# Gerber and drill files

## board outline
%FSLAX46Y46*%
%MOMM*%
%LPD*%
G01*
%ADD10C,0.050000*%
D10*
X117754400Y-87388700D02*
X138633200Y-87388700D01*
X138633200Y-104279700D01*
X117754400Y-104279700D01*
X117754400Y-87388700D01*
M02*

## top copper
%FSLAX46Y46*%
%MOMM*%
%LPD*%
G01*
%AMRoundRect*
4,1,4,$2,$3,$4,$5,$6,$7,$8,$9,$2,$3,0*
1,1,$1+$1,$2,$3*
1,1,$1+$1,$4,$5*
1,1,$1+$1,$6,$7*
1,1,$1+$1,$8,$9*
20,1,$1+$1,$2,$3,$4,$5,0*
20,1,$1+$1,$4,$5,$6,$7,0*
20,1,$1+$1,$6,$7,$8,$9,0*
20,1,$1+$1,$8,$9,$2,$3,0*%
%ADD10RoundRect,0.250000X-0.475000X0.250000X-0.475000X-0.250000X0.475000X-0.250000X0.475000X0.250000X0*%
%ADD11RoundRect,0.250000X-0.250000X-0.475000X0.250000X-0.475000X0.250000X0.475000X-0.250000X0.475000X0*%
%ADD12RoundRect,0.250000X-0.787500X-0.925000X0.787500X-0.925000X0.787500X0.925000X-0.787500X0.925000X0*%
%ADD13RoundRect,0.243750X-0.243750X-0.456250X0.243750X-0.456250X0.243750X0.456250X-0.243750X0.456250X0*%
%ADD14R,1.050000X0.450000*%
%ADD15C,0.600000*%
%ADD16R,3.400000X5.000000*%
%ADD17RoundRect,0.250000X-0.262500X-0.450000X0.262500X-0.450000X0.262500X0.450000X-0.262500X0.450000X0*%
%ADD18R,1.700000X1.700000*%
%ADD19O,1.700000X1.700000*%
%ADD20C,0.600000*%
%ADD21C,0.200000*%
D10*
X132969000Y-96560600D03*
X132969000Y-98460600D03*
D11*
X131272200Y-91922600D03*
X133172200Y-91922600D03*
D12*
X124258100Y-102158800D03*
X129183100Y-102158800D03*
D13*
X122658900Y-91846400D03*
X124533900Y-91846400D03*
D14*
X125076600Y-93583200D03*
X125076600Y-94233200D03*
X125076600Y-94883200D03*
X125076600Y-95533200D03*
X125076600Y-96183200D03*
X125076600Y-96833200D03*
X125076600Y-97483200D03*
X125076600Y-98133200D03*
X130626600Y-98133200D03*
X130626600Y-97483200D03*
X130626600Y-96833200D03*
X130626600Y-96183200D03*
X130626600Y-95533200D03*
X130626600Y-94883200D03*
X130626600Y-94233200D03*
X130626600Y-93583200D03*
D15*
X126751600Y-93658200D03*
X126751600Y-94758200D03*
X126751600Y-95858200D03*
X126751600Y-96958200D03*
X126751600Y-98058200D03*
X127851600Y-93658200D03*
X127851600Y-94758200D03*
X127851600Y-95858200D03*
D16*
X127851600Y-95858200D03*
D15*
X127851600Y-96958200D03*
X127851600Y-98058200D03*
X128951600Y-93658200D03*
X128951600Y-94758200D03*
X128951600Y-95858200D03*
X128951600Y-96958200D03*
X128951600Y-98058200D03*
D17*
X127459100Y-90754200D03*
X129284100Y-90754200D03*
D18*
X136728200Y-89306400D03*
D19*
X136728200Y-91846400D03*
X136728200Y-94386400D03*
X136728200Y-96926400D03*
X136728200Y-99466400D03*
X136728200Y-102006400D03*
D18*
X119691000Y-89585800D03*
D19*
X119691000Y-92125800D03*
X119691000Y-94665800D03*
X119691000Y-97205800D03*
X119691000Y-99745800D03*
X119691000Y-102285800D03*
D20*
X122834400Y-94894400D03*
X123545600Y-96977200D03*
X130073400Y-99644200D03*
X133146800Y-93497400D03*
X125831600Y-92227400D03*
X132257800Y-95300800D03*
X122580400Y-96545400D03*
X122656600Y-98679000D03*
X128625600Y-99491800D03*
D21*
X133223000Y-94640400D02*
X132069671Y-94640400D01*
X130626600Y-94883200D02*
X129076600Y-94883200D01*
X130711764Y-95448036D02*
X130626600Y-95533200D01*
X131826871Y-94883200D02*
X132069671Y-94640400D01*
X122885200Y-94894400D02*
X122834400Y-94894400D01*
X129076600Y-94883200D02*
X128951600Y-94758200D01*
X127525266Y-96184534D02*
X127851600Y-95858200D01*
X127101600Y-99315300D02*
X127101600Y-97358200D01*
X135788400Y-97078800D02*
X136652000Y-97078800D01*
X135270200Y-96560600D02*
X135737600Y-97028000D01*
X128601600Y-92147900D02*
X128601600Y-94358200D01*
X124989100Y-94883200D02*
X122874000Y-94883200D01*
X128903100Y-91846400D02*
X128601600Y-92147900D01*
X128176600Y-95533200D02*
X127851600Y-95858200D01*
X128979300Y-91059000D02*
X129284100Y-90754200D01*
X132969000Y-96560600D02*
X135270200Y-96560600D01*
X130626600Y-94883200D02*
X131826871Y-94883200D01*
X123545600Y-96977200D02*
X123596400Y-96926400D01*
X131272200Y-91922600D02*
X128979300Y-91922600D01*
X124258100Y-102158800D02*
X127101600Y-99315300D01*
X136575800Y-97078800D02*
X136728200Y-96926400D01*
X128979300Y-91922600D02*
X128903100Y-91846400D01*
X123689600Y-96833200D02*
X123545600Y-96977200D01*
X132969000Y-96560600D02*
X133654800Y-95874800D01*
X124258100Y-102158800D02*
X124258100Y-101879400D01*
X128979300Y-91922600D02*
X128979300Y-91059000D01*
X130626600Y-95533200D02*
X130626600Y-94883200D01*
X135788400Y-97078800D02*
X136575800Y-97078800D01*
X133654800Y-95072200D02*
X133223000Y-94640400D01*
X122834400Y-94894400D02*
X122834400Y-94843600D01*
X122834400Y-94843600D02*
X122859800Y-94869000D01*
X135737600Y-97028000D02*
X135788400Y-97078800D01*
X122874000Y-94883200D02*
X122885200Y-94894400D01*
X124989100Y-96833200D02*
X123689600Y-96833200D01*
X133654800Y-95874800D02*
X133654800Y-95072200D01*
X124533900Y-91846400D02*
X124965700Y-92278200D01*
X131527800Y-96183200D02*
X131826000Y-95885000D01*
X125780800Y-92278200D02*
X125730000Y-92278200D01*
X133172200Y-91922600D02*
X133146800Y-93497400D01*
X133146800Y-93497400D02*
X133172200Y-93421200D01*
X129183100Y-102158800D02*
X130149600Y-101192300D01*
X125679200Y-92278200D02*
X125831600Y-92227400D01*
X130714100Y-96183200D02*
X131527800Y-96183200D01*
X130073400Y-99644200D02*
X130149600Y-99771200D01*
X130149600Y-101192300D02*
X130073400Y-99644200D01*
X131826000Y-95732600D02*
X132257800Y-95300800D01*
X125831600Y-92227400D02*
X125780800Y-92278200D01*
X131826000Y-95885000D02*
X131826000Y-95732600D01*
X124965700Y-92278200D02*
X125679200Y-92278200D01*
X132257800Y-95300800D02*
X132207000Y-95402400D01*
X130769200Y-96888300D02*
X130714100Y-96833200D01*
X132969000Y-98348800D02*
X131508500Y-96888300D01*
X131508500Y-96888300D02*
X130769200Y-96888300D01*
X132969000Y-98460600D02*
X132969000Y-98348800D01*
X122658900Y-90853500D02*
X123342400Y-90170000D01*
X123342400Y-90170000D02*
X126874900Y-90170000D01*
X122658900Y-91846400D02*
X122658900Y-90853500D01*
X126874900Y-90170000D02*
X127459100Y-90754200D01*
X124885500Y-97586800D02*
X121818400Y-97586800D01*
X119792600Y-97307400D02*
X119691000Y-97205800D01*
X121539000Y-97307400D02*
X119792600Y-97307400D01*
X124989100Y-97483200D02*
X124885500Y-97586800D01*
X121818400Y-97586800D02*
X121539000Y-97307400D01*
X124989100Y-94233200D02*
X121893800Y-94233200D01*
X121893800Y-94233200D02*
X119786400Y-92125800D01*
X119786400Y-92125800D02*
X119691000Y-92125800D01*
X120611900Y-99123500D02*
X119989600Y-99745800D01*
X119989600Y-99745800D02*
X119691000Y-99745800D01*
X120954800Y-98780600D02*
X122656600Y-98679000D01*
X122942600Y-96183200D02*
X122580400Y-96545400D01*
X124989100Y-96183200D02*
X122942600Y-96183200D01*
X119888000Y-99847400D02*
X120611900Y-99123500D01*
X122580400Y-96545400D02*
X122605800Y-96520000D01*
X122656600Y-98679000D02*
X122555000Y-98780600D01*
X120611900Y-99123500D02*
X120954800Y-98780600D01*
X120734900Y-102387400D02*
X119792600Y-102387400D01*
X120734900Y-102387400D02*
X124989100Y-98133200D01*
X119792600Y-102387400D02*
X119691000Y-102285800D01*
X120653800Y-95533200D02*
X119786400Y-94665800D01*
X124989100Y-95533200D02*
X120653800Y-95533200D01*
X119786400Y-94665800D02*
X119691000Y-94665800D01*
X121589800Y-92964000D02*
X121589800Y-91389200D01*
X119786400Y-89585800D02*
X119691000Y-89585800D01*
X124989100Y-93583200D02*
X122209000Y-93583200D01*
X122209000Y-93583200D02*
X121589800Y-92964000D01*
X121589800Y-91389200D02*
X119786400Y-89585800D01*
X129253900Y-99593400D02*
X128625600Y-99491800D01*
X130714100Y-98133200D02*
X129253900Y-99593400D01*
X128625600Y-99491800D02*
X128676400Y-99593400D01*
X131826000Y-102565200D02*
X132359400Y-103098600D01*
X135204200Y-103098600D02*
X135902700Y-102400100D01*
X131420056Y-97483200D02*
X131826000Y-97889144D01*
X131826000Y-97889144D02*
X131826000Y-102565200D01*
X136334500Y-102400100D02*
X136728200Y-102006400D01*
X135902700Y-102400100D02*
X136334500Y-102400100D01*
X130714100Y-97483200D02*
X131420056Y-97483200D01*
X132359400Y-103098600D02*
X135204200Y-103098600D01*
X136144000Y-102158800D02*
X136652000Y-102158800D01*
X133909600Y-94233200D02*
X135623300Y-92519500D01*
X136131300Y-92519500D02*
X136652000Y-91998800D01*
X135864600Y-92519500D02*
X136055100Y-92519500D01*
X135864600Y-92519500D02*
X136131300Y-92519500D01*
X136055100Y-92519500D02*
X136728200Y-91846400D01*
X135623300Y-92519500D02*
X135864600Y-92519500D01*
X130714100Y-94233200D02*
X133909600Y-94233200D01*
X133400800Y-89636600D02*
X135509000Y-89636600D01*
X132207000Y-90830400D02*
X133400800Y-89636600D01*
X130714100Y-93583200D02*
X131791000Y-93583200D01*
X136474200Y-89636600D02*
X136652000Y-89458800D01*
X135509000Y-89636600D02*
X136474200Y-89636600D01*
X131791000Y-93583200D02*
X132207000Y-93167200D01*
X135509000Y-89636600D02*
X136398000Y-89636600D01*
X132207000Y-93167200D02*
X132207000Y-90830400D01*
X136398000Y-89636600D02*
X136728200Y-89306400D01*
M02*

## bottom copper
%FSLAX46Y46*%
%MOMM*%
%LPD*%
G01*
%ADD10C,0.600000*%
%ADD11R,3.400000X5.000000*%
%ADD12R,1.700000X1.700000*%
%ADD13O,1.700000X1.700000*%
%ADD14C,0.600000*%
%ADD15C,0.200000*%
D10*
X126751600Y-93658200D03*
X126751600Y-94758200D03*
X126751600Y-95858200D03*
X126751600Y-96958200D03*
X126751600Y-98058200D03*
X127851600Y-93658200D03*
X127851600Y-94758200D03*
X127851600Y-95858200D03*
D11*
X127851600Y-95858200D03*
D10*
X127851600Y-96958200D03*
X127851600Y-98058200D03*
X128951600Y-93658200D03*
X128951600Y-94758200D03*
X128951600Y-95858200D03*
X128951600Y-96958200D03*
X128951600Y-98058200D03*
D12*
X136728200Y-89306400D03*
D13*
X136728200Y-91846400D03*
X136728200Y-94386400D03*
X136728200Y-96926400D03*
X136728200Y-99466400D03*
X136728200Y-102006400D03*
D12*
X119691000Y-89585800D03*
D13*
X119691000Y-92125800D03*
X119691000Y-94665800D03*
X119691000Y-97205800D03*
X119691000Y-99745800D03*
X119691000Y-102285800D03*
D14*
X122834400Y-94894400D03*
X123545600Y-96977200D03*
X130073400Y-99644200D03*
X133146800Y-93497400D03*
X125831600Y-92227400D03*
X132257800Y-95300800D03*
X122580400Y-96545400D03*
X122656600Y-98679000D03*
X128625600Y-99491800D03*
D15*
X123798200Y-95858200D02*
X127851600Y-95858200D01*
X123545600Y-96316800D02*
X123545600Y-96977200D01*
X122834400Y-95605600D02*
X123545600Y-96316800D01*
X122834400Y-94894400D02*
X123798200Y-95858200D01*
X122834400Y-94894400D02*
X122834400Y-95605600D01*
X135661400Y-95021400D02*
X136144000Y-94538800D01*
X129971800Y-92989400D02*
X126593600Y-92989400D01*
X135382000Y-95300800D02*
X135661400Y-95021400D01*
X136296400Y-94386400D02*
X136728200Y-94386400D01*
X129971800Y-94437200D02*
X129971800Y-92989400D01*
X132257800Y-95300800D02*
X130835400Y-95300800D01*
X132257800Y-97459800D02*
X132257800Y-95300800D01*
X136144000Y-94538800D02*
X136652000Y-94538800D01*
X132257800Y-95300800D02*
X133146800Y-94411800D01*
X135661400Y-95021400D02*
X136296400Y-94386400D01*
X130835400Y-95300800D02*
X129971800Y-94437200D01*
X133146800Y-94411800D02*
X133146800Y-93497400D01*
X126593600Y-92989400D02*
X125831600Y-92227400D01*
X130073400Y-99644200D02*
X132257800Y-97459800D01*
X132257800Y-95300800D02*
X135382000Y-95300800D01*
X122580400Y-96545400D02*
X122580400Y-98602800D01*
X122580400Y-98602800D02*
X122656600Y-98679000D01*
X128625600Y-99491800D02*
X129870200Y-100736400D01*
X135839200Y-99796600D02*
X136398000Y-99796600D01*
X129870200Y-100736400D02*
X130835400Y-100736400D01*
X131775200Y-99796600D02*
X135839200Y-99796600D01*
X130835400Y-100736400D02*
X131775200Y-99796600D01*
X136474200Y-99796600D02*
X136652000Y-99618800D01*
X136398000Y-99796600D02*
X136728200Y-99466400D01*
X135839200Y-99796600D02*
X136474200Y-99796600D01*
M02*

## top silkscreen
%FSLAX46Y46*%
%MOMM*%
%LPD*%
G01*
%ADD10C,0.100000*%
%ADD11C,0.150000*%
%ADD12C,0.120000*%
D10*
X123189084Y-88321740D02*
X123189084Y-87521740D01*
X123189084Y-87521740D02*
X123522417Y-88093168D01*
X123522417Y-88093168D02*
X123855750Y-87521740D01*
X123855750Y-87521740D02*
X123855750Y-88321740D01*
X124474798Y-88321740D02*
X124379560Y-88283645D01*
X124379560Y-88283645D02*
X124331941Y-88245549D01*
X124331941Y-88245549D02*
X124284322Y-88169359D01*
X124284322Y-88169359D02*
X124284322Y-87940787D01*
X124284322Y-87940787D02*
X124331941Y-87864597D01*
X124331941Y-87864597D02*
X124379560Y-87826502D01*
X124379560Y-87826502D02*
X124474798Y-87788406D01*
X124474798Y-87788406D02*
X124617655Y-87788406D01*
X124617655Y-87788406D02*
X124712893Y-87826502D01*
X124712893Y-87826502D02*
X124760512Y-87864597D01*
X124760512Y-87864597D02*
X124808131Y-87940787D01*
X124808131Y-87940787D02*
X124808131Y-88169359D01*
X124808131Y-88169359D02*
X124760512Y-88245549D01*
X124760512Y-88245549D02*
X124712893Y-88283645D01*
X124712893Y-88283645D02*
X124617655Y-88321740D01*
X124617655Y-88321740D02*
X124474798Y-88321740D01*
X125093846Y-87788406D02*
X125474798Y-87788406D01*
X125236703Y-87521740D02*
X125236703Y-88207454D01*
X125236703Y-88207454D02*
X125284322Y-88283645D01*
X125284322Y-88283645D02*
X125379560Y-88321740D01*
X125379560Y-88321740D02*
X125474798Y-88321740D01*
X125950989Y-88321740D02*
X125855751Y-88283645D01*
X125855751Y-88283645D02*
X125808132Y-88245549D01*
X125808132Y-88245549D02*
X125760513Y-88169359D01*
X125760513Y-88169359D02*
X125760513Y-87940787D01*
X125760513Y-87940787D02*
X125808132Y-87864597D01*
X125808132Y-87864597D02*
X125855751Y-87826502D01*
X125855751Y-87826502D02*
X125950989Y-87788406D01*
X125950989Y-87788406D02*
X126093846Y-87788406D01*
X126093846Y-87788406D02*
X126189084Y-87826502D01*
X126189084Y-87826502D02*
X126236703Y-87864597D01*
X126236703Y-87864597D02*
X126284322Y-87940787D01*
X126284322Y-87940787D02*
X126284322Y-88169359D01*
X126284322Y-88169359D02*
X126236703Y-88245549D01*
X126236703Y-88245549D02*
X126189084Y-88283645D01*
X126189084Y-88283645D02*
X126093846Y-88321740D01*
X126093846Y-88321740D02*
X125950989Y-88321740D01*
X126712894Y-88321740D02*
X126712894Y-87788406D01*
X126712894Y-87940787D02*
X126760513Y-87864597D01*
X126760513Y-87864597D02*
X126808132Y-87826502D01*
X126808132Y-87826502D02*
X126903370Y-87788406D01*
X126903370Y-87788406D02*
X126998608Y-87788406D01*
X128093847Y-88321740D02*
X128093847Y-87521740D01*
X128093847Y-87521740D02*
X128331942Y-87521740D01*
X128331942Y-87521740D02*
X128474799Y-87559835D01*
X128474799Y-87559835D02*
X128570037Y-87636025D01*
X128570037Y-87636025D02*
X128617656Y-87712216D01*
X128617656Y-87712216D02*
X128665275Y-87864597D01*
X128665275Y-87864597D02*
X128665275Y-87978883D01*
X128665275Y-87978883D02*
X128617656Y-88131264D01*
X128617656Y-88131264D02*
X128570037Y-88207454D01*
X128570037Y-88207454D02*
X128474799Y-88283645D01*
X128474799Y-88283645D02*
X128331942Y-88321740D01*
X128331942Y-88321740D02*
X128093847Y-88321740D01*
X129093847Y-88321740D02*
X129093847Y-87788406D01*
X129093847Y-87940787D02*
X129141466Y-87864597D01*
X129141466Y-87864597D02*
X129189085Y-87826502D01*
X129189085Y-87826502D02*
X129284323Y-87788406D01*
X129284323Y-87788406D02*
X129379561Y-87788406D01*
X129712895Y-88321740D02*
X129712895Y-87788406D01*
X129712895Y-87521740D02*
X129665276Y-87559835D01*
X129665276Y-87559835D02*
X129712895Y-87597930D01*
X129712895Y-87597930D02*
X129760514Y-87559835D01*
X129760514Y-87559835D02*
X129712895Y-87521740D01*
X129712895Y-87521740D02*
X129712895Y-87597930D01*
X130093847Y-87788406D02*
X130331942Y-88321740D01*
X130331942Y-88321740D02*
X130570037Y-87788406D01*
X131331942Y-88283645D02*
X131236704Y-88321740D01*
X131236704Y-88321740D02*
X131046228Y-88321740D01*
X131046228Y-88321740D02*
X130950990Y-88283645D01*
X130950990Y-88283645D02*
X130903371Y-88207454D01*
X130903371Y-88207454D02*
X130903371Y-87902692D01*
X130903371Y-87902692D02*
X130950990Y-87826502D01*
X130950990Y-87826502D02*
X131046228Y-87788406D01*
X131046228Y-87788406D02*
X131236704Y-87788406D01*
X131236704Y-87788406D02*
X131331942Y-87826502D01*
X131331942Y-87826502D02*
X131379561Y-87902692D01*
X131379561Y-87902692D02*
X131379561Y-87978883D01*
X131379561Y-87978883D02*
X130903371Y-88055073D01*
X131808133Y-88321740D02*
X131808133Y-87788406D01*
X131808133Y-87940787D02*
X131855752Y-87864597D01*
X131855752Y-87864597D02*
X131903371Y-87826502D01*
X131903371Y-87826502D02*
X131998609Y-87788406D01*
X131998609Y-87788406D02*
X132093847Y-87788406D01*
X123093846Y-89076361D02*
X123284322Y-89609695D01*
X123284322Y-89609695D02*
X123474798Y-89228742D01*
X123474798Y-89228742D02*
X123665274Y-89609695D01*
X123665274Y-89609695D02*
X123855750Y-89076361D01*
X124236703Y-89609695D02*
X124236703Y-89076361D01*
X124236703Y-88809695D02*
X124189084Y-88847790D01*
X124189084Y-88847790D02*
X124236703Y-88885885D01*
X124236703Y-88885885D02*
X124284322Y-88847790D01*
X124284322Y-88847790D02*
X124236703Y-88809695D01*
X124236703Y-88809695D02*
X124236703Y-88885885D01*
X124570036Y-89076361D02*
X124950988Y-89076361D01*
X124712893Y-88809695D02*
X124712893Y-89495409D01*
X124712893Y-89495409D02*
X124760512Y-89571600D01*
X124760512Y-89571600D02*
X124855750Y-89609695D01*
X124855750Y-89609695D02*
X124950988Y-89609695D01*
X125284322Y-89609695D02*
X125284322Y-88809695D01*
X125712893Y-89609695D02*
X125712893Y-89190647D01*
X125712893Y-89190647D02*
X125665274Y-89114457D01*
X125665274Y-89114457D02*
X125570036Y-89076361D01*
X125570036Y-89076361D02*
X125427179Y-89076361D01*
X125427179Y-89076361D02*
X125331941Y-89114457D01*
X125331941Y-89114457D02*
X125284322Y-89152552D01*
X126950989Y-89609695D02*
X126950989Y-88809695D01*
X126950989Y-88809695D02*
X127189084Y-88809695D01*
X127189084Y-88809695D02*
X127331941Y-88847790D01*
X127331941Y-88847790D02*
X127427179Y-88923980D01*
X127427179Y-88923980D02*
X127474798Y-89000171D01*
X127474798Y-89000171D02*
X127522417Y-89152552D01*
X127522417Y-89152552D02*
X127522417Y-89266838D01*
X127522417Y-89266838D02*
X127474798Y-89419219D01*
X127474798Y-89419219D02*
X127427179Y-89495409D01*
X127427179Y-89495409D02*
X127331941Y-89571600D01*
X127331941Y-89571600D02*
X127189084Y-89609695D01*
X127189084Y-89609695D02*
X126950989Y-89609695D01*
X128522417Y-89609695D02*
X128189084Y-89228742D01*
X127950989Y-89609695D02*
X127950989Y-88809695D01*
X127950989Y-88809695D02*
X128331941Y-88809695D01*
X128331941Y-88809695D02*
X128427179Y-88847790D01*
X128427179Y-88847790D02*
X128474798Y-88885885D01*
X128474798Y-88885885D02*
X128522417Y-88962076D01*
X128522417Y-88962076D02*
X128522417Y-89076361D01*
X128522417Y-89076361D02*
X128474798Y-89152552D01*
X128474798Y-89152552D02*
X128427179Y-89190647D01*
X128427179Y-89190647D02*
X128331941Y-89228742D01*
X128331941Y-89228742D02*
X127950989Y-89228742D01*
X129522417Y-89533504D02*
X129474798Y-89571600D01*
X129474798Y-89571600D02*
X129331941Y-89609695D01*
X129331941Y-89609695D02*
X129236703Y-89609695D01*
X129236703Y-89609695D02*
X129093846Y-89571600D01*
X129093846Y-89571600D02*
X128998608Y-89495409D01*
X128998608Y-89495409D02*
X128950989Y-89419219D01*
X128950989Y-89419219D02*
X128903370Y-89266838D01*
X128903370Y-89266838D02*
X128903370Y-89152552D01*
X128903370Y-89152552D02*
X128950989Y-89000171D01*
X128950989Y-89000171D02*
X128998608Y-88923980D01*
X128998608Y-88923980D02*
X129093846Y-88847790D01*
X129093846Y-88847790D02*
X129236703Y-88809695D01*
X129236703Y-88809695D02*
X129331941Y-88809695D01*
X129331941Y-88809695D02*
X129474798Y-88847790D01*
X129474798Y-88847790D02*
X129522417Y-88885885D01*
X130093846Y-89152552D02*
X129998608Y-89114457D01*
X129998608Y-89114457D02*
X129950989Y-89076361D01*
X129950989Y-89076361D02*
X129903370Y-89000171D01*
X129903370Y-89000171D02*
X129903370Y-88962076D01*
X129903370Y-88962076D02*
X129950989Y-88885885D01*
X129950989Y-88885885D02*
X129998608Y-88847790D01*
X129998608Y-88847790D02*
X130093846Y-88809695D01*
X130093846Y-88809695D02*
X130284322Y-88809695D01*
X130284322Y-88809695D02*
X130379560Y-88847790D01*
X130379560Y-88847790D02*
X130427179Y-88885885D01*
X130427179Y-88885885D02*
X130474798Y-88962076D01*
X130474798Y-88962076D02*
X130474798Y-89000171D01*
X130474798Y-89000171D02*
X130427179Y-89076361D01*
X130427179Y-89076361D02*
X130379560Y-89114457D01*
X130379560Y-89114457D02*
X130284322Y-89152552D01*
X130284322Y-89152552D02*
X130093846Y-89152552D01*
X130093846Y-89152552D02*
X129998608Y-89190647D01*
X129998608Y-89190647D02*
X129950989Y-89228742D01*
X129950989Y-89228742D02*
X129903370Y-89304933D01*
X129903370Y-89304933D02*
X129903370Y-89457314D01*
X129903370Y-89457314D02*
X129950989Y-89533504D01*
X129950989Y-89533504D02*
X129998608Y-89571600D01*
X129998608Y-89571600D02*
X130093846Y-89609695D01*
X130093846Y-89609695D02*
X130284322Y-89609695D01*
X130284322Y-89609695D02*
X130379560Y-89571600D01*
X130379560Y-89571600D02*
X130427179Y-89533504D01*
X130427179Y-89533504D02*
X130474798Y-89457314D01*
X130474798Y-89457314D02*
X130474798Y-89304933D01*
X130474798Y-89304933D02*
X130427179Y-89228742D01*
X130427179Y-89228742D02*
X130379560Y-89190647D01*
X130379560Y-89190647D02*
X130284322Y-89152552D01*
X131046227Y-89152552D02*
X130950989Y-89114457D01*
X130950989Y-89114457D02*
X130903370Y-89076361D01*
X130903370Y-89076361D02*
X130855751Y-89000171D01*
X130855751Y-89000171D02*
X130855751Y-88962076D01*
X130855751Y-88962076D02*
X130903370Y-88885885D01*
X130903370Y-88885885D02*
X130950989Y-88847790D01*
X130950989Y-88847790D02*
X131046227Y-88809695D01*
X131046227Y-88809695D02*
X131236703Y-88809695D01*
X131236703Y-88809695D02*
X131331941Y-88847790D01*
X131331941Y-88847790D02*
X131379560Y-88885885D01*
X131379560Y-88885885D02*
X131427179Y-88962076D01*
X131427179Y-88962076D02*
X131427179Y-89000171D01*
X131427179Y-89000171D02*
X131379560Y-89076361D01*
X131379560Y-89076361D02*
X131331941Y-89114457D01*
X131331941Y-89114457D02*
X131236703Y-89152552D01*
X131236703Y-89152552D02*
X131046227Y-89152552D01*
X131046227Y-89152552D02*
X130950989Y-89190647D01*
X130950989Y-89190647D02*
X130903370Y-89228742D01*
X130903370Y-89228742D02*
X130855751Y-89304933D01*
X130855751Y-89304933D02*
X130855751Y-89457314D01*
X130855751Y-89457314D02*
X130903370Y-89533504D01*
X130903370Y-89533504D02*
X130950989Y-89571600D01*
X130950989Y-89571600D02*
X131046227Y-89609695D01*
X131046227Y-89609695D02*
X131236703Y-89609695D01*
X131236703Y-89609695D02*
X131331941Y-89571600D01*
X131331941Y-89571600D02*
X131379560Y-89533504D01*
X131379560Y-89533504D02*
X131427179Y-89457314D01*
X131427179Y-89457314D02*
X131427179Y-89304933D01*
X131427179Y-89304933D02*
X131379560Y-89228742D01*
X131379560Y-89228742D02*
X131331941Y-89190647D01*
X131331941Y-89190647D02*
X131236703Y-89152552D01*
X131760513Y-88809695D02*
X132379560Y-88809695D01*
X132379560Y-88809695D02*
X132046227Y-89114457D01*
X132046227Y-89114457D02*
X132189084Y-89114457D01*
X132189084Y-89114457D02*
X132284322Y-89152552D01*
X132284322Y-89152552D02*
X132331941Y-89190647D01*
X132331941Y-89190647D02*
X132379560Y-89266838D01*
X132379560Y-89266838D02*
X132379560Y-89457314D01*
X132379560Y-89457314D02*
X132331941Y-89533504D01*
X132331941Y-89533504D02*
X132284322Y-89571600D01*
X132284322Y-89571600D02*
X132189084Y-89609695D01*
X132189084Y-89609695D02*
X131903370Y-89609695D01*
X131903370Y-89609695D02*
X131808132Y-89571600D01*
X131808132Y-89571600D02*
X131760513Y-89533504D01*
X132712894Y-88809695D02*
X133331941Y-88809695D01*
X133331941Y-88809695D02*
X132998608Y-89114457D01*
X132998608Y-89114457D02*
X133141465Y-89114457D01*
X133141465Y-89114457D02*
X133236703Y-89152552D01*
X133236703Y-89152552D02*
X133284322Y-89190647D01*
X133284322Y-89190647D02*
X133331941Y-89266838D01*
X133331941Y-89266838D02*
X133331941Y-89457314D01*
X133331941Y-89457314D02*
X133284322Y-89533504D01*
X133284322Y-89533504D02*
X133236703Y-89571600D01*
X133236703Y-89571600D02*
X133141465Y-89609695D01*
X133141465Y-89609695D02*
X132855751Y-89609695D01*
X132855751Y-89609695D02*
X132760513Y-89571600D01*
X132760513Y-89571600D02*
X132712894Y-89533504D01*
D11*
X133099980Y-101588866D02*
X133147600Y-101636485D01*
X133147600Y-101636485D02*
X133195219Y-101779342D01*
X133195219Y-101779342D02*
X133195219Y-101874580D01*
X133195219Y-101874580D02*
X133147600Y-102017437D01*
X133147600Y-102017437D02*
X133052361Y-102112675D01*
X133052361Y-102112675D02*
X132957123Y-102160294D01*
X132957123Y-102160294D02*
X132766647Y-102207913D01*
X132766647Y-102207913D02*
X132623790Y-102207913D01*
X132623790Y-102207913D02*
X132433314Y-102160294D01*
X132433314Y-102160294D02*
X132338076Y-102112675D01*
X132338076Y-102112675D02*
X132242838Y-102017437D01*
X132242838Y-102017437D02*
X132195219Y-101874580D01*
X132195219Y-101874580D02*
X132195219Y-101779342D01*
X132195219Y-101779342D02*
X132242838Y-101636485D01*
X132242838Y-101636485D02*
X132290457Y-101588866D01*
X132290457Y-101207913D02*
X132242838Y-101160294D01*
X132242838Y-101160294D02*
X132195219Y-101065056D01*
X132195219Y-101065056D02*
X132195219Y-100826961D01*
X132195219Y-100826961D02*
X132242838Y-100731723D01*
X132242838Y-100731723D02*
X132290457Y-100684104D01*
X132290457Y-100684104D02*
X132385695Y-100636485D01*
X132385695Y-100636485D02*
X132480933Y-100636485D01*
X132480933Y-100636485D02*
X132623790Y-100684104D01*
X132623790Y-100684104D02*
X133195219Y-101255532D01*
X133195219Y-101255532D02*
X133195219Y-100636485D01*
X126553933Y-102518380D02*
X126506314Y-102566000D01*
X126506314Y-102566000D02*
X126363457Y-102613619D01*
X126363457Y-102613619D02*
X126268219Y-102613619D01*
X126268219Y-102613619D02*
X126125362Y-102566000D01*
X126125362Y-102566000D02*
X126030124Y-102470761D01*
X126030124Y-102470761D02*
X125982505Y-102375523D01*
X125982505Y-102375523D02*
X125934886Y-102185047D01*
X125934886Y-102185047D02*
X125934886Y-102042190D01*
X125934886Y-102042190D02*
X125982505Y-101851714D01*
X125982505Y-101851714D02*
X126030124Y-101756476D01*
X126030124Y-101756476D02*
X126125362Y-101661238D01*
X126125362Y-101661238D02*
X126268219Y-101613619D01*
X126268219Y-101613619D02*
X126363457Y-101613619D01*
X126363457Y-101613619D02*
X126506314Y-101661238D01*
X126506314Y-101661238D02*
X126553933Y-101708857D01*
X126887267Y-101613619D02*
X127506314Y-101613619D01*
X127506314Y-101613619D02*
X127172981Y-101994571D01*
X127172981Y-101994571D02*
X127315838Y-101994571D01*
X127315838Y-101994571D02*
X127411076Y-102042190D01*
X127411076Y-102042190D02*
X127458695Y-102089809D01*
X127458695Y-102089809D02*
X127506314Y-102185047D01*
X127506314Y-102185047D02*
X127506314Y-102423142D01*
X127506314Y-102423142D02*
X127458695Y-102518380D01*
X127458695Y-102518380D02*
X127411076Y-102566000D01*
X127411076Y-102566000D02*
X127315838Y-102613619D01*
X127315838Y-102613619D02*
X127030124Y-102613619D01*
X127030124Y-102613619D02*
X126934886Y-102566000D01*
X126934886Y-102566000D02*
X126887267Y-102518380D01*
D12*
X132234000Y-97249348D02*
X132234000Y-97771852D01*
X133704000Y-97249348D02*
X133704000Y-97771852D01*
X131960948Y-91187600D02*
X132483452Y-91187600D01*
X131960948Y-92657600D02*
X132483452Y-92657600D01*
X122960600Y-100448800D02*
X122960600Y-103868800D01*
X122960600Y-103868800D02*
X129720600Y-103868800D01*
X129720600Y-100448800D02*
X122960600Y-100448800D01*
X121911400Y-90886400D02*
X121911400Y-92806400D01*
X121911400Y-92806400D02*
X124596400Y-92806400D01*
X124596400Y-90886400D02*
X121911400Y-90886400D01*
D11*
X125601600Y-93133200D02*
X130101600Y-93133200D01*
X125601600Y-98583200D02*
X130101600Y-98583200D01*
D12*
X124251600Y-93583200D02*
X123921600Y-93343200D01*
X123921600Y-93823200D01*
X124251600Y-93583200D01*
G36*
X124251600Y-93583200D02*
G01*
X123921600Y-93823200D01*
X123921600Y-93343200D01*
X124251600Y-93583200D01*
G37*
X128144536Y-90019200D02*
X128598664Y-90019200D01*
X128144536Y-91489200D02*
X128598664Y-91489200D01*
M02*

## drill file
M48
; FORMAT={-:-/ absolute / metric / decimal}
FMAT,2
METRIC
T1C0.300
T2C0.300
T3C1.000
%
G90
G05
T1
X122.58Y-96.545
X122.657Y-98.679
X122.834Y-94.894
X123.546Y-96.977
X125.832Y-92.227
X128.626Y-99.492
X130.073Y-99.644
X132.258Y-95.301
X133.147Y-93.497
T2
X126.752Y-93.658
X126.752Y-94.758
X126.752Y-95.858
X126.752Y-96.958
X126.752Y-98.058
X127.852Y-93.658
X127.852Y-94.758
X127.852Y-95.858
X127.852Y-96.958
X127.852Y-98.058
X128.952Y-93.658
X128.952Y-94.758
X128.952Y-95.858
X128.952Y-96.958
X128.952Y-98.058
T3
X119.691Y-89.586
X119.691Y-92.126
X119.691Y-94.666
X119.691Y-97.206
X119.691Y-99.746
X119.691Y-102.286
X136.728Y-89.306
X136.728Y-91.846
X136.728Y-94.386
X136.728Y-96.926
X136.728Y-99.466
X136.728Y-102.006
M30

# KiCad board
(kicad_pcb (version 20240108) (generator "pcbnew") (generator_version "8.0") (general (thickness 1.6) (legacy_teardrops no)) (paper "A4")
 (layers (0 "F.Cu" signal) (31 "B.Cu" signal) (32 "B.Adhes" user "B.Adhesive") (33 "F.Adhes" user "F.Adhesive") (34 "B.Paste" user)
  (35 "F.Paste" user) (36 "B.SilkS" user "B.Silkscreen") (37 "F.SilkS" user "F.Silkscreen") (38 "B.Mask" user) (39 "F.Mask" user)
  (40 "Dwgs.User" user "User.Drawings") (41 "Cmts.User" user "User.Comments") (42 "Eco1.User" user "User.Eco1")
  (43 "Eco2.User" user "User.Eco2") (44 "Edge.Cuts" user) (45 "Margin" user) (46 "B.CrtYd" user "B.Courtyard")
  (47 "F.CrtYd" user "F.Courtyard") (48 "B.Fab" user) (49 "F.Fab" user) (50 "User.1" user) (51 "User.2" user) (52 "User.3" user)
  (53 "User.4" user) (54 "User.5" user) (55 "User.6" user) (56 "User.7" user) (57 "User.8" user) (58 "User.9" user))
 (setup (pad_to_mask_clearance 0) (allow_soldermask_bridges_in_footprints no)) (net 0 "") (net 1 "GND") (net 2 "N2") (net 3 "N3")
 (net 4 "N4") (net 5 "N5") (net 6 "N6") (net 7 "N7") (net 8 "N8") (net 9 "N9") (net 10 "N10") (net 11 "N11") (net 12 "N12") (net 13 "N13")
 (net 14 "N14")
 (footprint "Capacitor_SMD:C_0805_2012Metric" (layer "F.Cu") (at 132.969 97.5106 -90)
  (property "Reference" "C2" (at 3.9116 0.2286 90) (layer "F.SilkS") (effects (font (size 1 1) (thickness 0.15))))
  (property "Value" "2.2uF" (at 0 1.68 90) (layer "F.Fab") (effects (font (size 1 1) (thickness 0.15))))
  (fp_line (start -0.261252 0.735) (end 0.261252 0.735) (stroke (width 0.12) (type solid)) (layer "F.SilkS"))
  (fp_line (start -0.261252 -0.735) (end 0.261252 -0.735) (stroke (width 0.12) (type solid)) (layer "F.SilkS"))
  (pad "1" smd roundrect (at -0.95 0 270) (size 1 1.45) (layers "F.Cu" "F.Paste" "F.Mask") (roundrect_rratio 0.25) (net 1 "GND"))
  (pad "2" smd roundrect (at 0.95 0 270) (size 1 1.45) (layers "F.Cu" "F.Paste" "F.Mask") (roundrect_rratio 0.25) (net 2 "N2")))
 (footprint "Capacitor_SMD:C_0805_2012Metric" (layer "F.Cu") (at 132.2222 91.9226)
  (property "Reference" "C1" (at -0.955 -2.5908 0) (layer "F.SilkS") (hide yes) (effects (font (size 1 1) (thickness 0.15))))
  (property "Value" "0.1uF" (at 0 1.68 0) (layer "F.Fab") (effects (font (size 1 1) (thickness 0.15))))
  (fp_line (start -0.261252 -0.735) (end 0.261252 -0.735) (stroke (width 0.12) (type solid)) (layer "F.SilkS"))
  (fp_line (start -0.261252 0.735) (end 0.261252 0.735) (stroke (width 0.12) (type solid)) (layer "F.SilkS"))
  (pad "1" smd roundrect (at -0.95 0) (size 1 1.45) (layers "F.Cu" "F.Paste" "F.Mask") (roundrect_rratio 0.25) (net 1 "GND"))
  (pad "2" smd roundrect (at 0.95 0) (size 1 1.45) (layers "F.Cu" "F.Paste" "F.Mask") (roundrect_rratio 0.25) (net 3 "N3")))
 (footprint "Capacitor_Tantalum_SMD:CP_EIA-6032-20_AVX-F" (layer "F.Cu") (at 126.7206 102.1588)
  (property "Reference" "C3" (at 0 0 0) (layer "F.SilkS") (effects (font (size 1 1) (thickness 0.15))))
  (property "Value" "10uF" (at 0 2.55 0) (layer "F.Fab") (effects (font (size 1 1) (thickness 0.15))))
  (fp_line (start -3.76 -1.71) (end -3.76 1.71) (stroke (width 0.12) (type solid)) (layer "F.SilkS"))
  (fp_line (start -3.76 1.71) (end 3 1.71) (stroke (width 0.12) (type solid)) (layer "F.SilkS"))
  (fp_line (start 3 -1.71) (end -3.76 -1.71) (stroke (width 0.12) (type solid)) (layer "F.SilkS"))
  (pad "1" smd roundrect (at -2.4625 0) (size 2.075 2.35) (layers "F.Cu" "F.Paste" "F.Mask") (roundrect_rratio 0.120482) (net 1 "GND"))
  (pad "2" smd roundrect (at 2.4625 0) (size 2.075 2.35) (layers "F.Cu" "F.Paste" "F.Mask") (roundrect_rratio 0.120482) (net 3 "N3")))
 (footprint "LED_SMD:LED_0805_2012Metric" (layer "F.Cu") (at 123.5964 91.8464)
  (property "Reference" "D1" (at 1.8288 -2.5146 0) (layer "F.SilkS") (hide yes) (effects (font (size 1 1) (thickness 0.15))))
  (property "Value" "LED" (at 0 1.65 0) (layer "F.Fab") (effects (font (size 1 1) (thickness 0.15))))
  (fp_line (start -1.685 -0.96) (end -1.685 0.96) (stroke (width 0.12) (type solid)) (layer "F.SilkS"))
  (fp_line (start -1.685 0.96) (end 1 0.96) (stroke (width 0.12) (type solid)) (layer "F.SilkS"))
  (fp_line (start 1 -0.96) (end -1.685 -0.96) (stroke (width 0.12) (type solid)) (layer "F.SilkS"))
  (pad "1" smd roundrect (at -0.9375 0) (size 0.975 1.4) (layers "F.Cu" "F.Paste" "F.Mask") (roundrect_rratio 0.25) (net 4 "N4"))
  (pad "2" smd roundrect (at 0.9375 0) (size 0.975 1.4) (layers "F.Cu" "F.Paste" "F.Mask") (roundrect_rratio 0.25) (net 3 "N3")))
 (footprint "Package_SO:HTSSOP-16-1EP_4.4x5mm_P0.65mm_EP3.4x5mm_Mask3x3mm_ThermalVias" (layer "F.Cu") (at 127.8516 95.8582)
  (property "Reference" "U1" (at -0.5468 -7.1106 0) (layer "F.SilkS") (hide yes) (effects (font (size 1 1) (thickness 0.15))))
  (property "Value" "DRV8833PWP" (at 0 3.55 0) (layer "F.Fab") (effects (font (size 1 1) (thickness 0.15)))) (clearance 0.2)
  (fp_line (start -2.25 -2.725) (end 2.25 -2.725) (stroke (width 0.15) (type solid)) (layer "F.SilkS"))
  (fp_line (start -2.25 2.725) (end 2.25 2.725) (stroke (width 0.15) (type solid)) (layer "F.SilkS"))
  (fp_poly
   (pts (xy -3.6 -2.275) (xy -3.93 -2.515) (xy -3.93 -2.035) (xy -3.6 -2.275)) (stroke (width 0.12) (type solid)) (fill solid)
   (layer "F.SilkS"))
  (pad "" smd rect (at -1.325 -0.55 90) (size 0.8 0.25) (layers "F.Paste"))
  (pad "" smd rect (at -1.325 0.55 90) (size 0.8 0.25) (layers "F.Paste"))
  (pad "" smd rect (at -0.55 -1.325) (size 0.8 0.25) (layers "F.Paste"))
  (pad "" smd rect (at -0.55 -0.55) (size 0.85 0.8) (layers "F.Paste"))
  (pad "" smd rect (at -0.55 0.55) (size 0.85 0.85) (layers "F.Paste"))
  (pad "" smd rect (at -0.55 1.325) (size 0.8 0.25) (layers "F.Paste")) (pad "" smd rect (at 0 0) (size 3 3) (layers "F.Mask"))
  (pad "" smd rect (at 0.55 -1.325) (size 0.8 0.25) (layers "F.Paste"))
  (pad "" smd rect (at 0.55 -0.55) (size 0.85 0.85) (layers "F.Paste"))
  (pad "" smd rect (at 0.55 0.55) (size 0.85 0.85) (layers "F.Paste"))
  (pad "" smd rect (at 0.55 1.325) (size 0.8 0.25) (layers "F.Paste"))
  (pad "" smd rect (at 1.325 -0.55 90) (size 0.8 0.25) (layers "F.Paste"))
  (pad "" smd rect (at 1.325 0.55 90) (size 0.8 0.25) (layers "F.Paste"))
  (pad "1" smd rect (at -2.775 -2.275) (size 1.05 0.45) (layers "F.Cu" "F.Paste" "F.Mask") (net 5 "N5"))
  (pad "2" smd rect (at -2.775 -1.625) (size 1.05 0.45) (layers "F.Cu" "F.Paste" "F.Mask") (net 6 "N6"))
  (pad "3" smd rect (at -2.775 -0.975) (size 1.05 0.45) (layers "F.Cu" "F.Paste" "F.Mask") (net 1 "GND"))
  (pad "4" smd rect (at -2.775 -0.325) (size 1.05 0.45) (layers "F.Cu" "F.Paste" "F.Mask") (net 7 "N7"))
  (pad "5" smd rect (at -2.775 0.325) (size 1.05 0.45) (layers "F.Cu" "F.Paste" "F.Mask") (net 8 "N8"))
  (pad "6" smd rect (at -2.775 0.975) (size 1.05 0.45) (layers "F.Cu" "F.Paste" "F.Mask") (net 1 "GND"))
  (pad "7" smd rect (at -2.775 1.625) (size 1.05 0.45) (layers "F.Cu" "F.Paste" "F.Mask") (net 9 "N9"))
  (pad "8" smd rect (at -2.775 2.275) (size 1.05 0.45) (layers "F.Cu" "F.Paste" "F.Mask") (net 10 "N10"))
  (pad "9" smd rect (at 2.775 2.275) (size 1.05 0.45) (layers "F.Cu" "F.Paste" "F.Mask") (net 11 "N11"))
  (pad "10" smd rect (at 2.775 1.625) (size 1.05 0.45) (layers "F.Cu" "F.Paste" "F.Mask") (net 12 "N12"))
  (pad "11" smd rect (at 2.775 0.975) (size 1.05 0.45) (layers "F.Cu" "F.Paste" "F.Mask") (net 2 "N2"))
  (pad "12" smd rect (at 2.775 0.325) (size 1.05 0.45) (layers "F.Cu" "F.Paste" "F.Mask") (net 3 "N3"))
  (pad "13" smd rect (at 2.775 -0.325) (size 1.05 0.45) (layers "F.Cu" "F.Paste" "F.Mask") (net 1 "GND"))
  (pad "14" smd rect (at 2.775 -0.975) (size 1.05 0.45) (layers "F.Cu" "F.Paste" "F.Mask") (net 1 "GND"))
  (pad "15" smd rect (at 2.775 -1.625) (size 1.05 0.45) (layers "F.Cu" "F.Paste" "F.Mask") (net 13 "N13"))
  (pad "16" smd rect (at 2.775 -2.275) (size 1.05 0.45) (layers "F.Cu" "F.Paste" "F.Mask") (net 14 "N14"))
  (pad "17" thru_hole circle (at -1.1 -2.2) (size 0.6 0.6) (drill 0.3) (layers "*.Cu") (remove_unused_layers no) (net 1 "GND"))
  (pad "17" thru_hole circle (at -1.1 -1.1) (size 0.6 0.6) (drill 0.3) (layers "*.Cu") (remove_unused_layers no) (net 1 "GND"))
  (pad "17" thru_hole circle (at -1.1 0) (size 0.6 0.6) (drill 0.3) (layers "*.Cu") (remove_unused_layers no) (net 1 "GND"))
  (pad "17" thru_hole circle (at -1.1 1.1) (size 0.6 0.6) (drill 0.3) (layers "*.Cu") (remove_unused_layers no) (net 1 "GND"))
  (pad "17" thru_hole circle (at -1.1 2.2) (size 0.6 0.6) (drill 0.3) (layers "*.Cu") (remove_unused_layers no) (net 1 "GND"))
  (pad "17" thru_hole circle (at 0 -2.2) (size 0.6 0.6) (drill 0.3) (layers "*.Cu") (remove_unused_layers no) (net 1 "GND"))
  (pad "17" thru_hole circle (at 0 -1.1) (size 0.6 0.6) (drill 0.3) (layers "*.Cu") (remove_unused_layers no) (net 1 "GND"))
  (pad "17" thru_hole circle (at 0 0) (size 0.6 0.6) (drill 0.3) (layers "*.Cu") (remove_unused_layers no) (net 1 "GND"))
  (pad "17" smd rect (at 0 0) (size 3.4 5) (layers "F.Cu") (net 1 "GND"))
  (pad "17" smd rect (at 0 0) (size 3.4 5) (layers "B.Cu") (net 1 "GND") (solder_paste_margin_ratio -0.2))
  (pad "17" thru_hole circle (at 0 1.1) (size 0.6 0.6) (drill 0.3) (layers "*.Cu") (remove_unused_layers no) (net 1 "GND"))
  (pad "17" thru_hole circle (at 0 2.2) (size 0.6 0.6) (drill 0.3) (layers "*.Cu") (remove_unused_layers no) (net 1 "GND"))
  (pad "17" thru_hole circle (at 1.1 -2.2) (size 0.6 0.6) (drill 0.3) (layers "*.Cu") (remove_unused_layers no) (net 1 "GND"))
  (pad "17" thru_hole circle (at 1.1 -1.1) (size 0.6 0.6) (drill 0.3) (layers "*.Cu") (remove_unused_layers no) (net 1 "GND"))
  (pad "17" thru_hole circle (at 1.1 0) (size 0.6 0.6) (drill 0.3) (layers "*.Cu") (remove_unused_layers no) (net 1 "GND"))
  (pad "17" thru_hole circle (at 1.1 1.1) (size 0.6 0.6) (drill 0.3) (layers "*.Cu") (remove_unused_layers no) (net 1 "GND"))
  (pad "17" thru_hole circle (at 1.1 2.2) (size 0.6 0.6) (drill 0.3) (layers "*.Cu") (remove_unused_layers no) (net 1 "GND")))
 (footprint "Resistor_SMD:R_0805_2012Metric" (layer "F.Cu") (at 128.3716 90.7542)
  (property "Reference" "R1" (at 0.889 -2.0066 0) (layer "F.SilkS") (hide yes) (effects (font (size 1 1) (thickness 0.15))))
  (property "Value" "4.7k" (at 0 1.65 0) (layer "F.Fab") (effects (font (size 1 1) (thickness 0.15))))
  (fp_line (start -0.227064 -0.735) (end 0.227064 -0.735) (stroke (width 0.12) (type solid)) (layer "F.SilkS"))
  (fp_line (start -0.227064 0.735) (end 0.227064 0.735) (stroke (width 0.12) (type solid)) (layer "F.SilkS"))
  (pad "1" smd roundrect (at -0.9125 0) (size 1.025 1.4) (layers "F.Cu" "F.Paste" "F.Mask") (roundrect_rratio 0.243902) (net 4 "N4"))
  (pad "2" smd roundrect (at 0.9125 0) (size 1.025 1.4) (layers "F.Cu" "F.Paste" "F.Mask") (roundrect_rratio 0.243902) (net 1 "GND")))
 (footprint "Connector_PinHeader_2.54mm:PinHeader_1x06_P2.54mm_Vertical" (layer "B.Cu") (at 136.7282 89.3064 180)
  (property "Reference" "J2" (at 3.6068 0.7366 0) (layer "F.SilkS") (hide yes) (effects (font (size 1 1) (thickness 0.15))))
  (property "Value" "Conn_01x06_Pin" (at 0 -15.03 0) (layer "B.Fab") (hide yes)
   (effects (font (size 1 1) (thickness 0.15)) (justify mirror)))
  (pad "1" thru_hole rect (at 0 0 180) (size 1.7 1.7) (drill 1) (layers "*.Cu" "*.Mask") (remove_unused_layers no) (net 14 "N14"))
  (pad "2" thru_hole oval (at 0 -2.54 180) (size 1.7 1.7) (drill 1) (layers "*.Cu" "*.Mask") (remove_unused_layers no) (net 13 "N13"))
  (pad "3" thru_hole oval (at 0 -5.08 180) (size 1.7 1.7) (drill 1) (layers "*.Cu" "*.Mask") (remove_unused_layers no) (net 3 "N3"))
  (pad "4" thru_hole oval (at 0 -7.62 180) (size 1.7 1.7) (drill 1) (layers "*.Cu" "*.Mask") (remove_unused_layers no) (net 1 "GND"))
  (pad "5" thru_hole oval (at 0 -10.16 180) (size 1.7 1.7) (drill 1) (layers "*.Cu" "*.Mask") (remove_unused_layers no) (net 11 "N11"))
  (pad "6" thru_hole oval (at 0 -12.7 180) (size 1.7 1.7) (drill 1) (layers "*.Cu" "*.Mask") (remove_unused_layers no) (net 12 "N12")))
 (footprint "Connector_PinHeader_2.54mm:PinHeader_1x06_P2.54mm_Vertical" (layer "B.Cu") (at 119.691 89.5858 180)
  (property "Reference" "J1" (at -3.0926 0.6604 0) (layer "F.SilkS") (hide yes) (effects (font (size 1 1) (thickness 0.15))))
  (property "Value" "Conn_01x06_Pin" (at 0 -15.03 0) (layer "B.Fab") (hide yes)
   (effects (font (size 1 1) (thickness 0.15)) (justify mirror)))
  (pad "1" thru_hole rect (at 0 0 180) (size 1.7 1.7) (drill 1) (layers "*.Cu" "*.Mask") (remove_unused_layers no) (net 5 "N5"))
  (pad "2" thru_hole oval (at 0 -2.54 180) (size 1.7 1.7) (drill 1) (layers "*.Cu" "*.Mask") (remove_unused_layers no) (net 6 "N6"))
  (pad "3" thru_hole oval (at 0 -5.08 180) (size 1.7 1.7) (drill 1) (layers "*.Cu" "*.Mask") (remove_unused_layers no) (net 7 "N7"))
  (pad "4" thru_hole oval (at 0 -7.62 180) (size 1.7 1.7) (drill 1) (layers "*.Cu" "*.Mask") (remove_unused_layers no) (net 9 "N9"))
  (pad "5" thru_hole oval (at 0 -10.16 180) (size 1.7 1.7) (drill 1) (layers "*.Cu" "*.Mask") (remove_unused_layers no) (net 8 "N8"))
  (pad "6" thru_hole oval (at 0 -12.7 180) (size 1.7 1.7) (drill 1) (layers "*.Cu" "*.Mask") (remove_unused_layers no) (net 10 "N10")))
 (gr_rect (start 117.7544 87.3887) (end 138.6332 104.2797) (stroke (width 0.05) (type default)) (fill none) (layer "Edge.Cuts"))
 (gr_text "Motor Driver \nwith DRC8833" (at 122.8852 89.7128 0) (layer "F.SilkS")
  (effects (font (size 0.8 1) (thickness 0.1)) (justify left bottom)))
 (segment (start 133.223 94.6404) (end 132.069671 94.6404) (width 0.2) (layer "F.Cu") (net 1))
 (segment (start 130.6266 94.8832) (end 129.0766 94.8832) (width 0.2) (layer "F.Cu") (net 1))
 (segment (start 130.711764 95.448036) (end 130.6266 95.5332) (width 0.2) (layer "F.Cu") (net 1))
 (segment (start 131.826871 94.8832) (end 132.069671 94.6404) (width 0.2) (layer "F.Cu") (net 1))
 (segment (start 122.8852 94.8944) (end 122.8344 94.8944) (width 0.2) (layer "F.Cu") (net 1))
 (segment (start 129.0766 94.8832) (end 128.9516 94.7582) (width 0.2) (layer "F.Cu") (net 1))
 (segment (start 127.525266 96.184534) (end 127.8516 95.8582) (width 0.2) (layer "F.Cu") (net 1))
 (segment (start 127.1016 99.3153) (end 127.1016 97.3582) (width 0.2) (layer "F.Cu") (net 1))
 (segment (start 135.7884 97.0788) (end 136.652 97.0788) (width 0.2) (layer "F.Cu") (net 1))
 (segment (start 135.2702 96.5606) (end 135.7376 97.028) (width 0.2) (layer "F.Cu") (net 1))
 (segment (start 128.6016 92.1479) (end 128.6016 94.3582) (width 0.2) (layer "F.Cu") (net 1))
 (segment (start 124.9891 94.8832) (end 122.874 94.8832) (width 0.2) (layer "F.Cu") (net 1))
 (segment (start 128.9031 91.8464) (end 128.6016 92.1479) (width 0.2) (layer "F.Cu") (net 1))
 (segment (start 128.1766 95.5332) (end 127.8516 95.8582) (width 0.2) (layer "F.Cu") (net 1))
 (segment (start 128.9793 91.059) (end 129.2841 90.7542) (width 0.2) (layer "F.Cu") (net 1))
 (segment (start 132.969 96.5606) (end 135.2702 96.5606) (width 0.2) (layer "F.Cu") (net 1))
 (segment (start 130.6266 94.8832) (end 131.826871 94.8832) (width 0.2) (layer "F.Cu") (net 1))
 (segment (start 123.5456 96.9772) (end 123.5964 96.9264) (width 0.2) (layer "F.Cu") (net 1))
 (segment (start 131.2722 91.9226) (end 128.9793 91.9226) (width 0.2) (layer "F.Cu") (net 1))
 (segment (start 124.2581 102.1588) (end 127.1016 99.3153) (width 0.2) (layer "F.Cu") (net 1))
 (segment (start 136.5758 97.0788) (end 136.7282 96.9264) (width 0.2) (layer "F.Cu") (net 1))
 (segment (start 128.9793 91.9226) (end 128.9031 91.8464) (width 0.2) (layer "F.Cu") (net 1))
 (segment (start 123.6896 96.8332) (end 123.5456 96.9772) (width 0.2) (layer "F.Cu") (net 1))
 (segment (start 132.969 96.5606) (end 133.6548 95.8748) (width 0.2) (layer "F.Cu") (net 1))
 (segment (start 124.2581 102.1588) (end 124.2581 101.8794) (width 0.2) (layer "F.Cu") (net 1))
 (segment (start 128.9793 91.9226) (end 128.9793 91.059) (width 0.2) (layer "F.Cu") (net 1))
 (segment (start 130.6266 95.5332) (end 130.6266 94.8832) (width 0.2) (layer "F.Cu") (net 1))
 (segment (start 135.7884 97.0788) (end 136.5758 97.0788) (width 0.2) (layer "F.Cu") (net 1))
 (segment (start 133.6548 95.0722) (end 133.223 94.6404) (width 0.2) (layer "F.Cu") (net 1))
 (segment (start 122.8344 94.8944) (end 122.8344 94.8436) (width 0.2) (layer "F.Cu") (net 1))
 (segment (start 122.8344 94.8436) (end 122.8598 94.869) (width 0.2) (layer "F.Cu") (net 1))
 (segment (start 135.7376 97.028) (end 135.7884 97.0788) (width 0.2) (layer "F.Cu") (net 1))
 (segment (start 122.874 94.8832) (end 122.8852 94.8944) (width 0.2) (layer "F.Cu") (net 1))
 (segment (start 124.9891 96.8332) (end 123.6896 96.8332) (width 0.2) (layer "F.Cu") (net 1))
 (segment (start 133.6548 95.8748) (end 133.6548 95.0722) (width 0.2) (layer "F.Cu") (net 1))
 (via (at 122.8344 94.8944) (size 0.6) (drill 0.3) (layers "F.Cu" "B.Cu") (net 1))
 (via (at 123.5456 96.9772) (size 0.6) (drill 0.3) (layers "F.Cu" "B.Cu") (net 1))
 (segment (start 123.7982 95.8582) (end 127.8516 95.8582) (width 0.2) (layer "B.Cu") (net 1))
 (segment (start 123.5456 96.3168) (end 123.5456 96.9772) (width 0.2) (layer "B.Cu") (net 1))
 (segment (start 122.8344 95.6056) (end 123.5456 96.3168) (width 0.2) (layer "B.Cu") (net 1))
 (segment (start 122.8344 94.8944) (end 123.7982 95.8582) (width 0.2) (layer "B.Cu") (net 1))
 (segment (start 122.8344 94.8944) (end 122.8344 95.6056) (width 0.2) (layer "B.Cu") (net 1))
 (segment (start 124.5339 91.8464) (end 124.9657 92.2782) (width 0.2) (layer "F.Cu") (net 3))
 (segment (start 131.5278 96.1832) (end 131.826 95.885) (width 0.2) (layer "F.Cu") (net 3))
 (segment (start 125.7808 92.2782) (end 125.73 92.2782) (width 0.2) (layer "F.Cu") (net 3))
 (segment (start 133.1722 91.9226) (end 133.1468 93.4974) (width 0.2) (layer "F.Cu") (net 3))
 (segment (start 133.1468 93.4974) (end 133.1722 93.4212) (width 0.2) (layer "F.Cu") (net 3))
 (segment (start 129.1831 102.1588) (end 130.1496 101.1923) (width 0.2) (layer "F.Cu") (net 3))
 (segment (start 125.6792 92.2782) (end 125.8316 92.2274) (width 0.2) (layer "F.Cu") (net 3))
 (segment (start 130.7141 96.1832) (end 131.5278 96.1832) (width 0.2) (layer "F.Cu") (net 3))
 (segment (start 130.0734 99.6442) (end 130.1496 99.7712) (width 0.2) (layer "F.Cu") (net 3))
 (segment (start 130.1496 101.1923) (end 130.0734 99.6442) (width 0.2) (layer "F.Cu") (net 3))
 (segment (start 131.826 95.7326) (end 132.2578 95.3008) (width 0.2) (layer "F.Cu") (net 3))
 (segment (start 125.8316 92.2274) (end 125.7808 92.2782) (width 0.2) (layer "F.Cu") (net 3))
 (segment (start 131.826 95.885) (end 131.826 95.7326) (width 0.2) (layer "F.Cu") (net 3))
 (segment (start 124.9657 92.2782) (end 125.6792 92.2782) (width 0.2) (layer "F.Cu") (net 3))
 (segment (start 132.2578 95.3008) (end 132.207 95.4024) (width 0.2) (layer "F.Cu") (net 3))
 (via (at 130.0734 99.6442) (size 0.6) (drill 0.3) (layers "F.Cu" "B.Cu") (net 3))
 (via (at 133.1468 93.4974) (size 0.6) (drill 0.3) (layers "F.Cu" "B.Cu") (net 3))
 (via (at 125.8316 92.2274) (size 0.6) (drill 0.3) (layers "F.Cu" "B.Cu") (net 3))
 (via (at 132.2578 95.3008) (size 0.6) (drill 0.3) (layers "F.Cu" "B.Cu") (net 3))
 (segment (start 135.6614 95.0214) (end 136.144 94.5388) (width 0.2) (layer "B.Cu") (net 3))
 (segment (start 129.9718 92.9894) (end 126.5936 92.9894) (width 0.2) (layer "B.Cu") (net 3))
 (segment (start 135.382 95.3008) (end 135.6614 95.0214) (width 0.2) (layer "B.Cu") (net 3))
 (segment (start 136.2964 94.3864) (end 136.7282 94.3864) (width 0.2) (layer "B.Cu") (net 3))
 (segment (start 129.9718 94.4372) (end 129.9718 92.9894) (width 0.2) (layer "B.Cu") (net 3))
 (segment (start 132.2578 95.3008) (end 130.8354 95.3008) (width 0.2) (layer "B.Cu") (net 3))
 (segment (start 132.2578 97.4598) (end 132.2578 95.3008) (width 0.2) (layer "B.Cu") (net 3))
 (segment (start 136.144 94.5388) (end 136.652 94.5388) (width 0.2) (layer "B.Cu") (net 3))
 (segment (start 132.2578 95.3008) (end 133.1468 94.4118) (width 0.2) (layer "B.Cu") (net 3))
 (segment (start 135.6614 95.0214) (end 136.2964 94.3864) (width 0.2) (layer "B.Cu") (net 3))
 (segment (start 130.8354 95.3008) (end 129.9718 94.4372) (width 0.2) (layer "B.Cu") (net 3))
 (segment (start 133.1468 94.4118) (end 133.1468 93.4974) (width 0.2) (layer "B.Cu") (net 3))
 (segment (start 126.5936 92.9894) (end 125.8316 92.2274) (width 0.2) (layer "B.Cu") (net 3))
 (segment (start 130.0734 99.6442) (end 132.2578 97.4598) (width 0.2) (layer "B.Cu") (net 3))
 (segment (start 132.2578 95.3008) (end 135.382 95.3008) (width 0.2) (layer "B.Cu") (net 3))
 (segment (start 130.7692 96.8883) (end 130.7141 96.8332) (width 0.2) (layer "F.Cu") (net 2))
 (segment (start 132.969 98.3488) (end 131.5085 96.8883) (width 0.2) (layer "F.Cu") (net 2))
 (segment (start 131.5085 96.8883) (end 130.7692 96.8883) (width 0.2) (layer "F.Cu") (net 2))
 (segment (start 132.969 98.4606) (end 132.969 98.3488) (width 0.2) (layer "F.Cu") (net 2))
 (segment (start 122.6589 90.8535) (end 123.3424 90.17) (width 0.2) (layer "F.Cu") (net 4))
 (segment (start 123.3424 90.17) (end 126.8749 90.17) (width 0.2) (layer "F.Cu") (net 4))
 (segment (start 122.6589 91.8464) (end 122.6589 90.8535) (width 0.2) (layer "F.Cu") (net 4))
 (segment (start 126.8749 90.17) (end 127.4591 90.7542) (width 0.2) (layer "F.Cu") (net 4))
 (segment (start 124.8855 97.5868) (end 121.8184 97.5868) (width 0.2) (layer "F.Cu") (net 9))
 (segment (start 119.7926 97.3074) (end 119.691 97.2058) (width 0.2) (layer "F.Cu") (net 9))
 (segment (start 121.539 97.3074) (end 119.7926 97.3074) (width 0.2) (layer "F.Cu") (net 9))
 (segment (start 124.9891 97.4832) (end 124.8855 97.5868) (width 0.2) (layer "F.Cu") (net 9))
 (segment (start 121.8184 97.5868) (end 121.539 97.3074) (width 0.2) (layer "F.Cu") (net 9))
 (segment (start 124.9891 94.2332) (end 121.8938 94.2332) (width 0.2) (layer "F.Cu") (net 6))
 (segment (start 121.8938 94.2332) (end 119.7864 92.1258) (width 0.2) (layer "F.Cu") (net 6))
 (segment (start 119.7864 92.1258) (end 119.691 92.1258) (width 0.2) (layer "F.Cu") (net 6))
 (segment (start 120.6119 99.1235) (end 119.9896 99.7458) (width 0.2) (layer "F.Cu") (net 8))
 (segment (start 119.9896 99.7458) (end 119.691 99.7458) (width 0.2) (layer "F.Cu") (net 8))
 (segment (start 120.9548 98.7806) (end 122.6566 98.679) (width 0.2) (layer "F.Cu") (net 8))
 (segment (start 122.9426 96.1832) (end 122.5804 96.5454) (width 0.2) (layer "F.Cu") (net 8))
 (segment (start 124.9891 96.1832) (end 122.9426 96.1832) (width 0.2) (layer "F.Cu") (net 8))
 (segment (start 119.888 99.8474) (end 120.6119 99.1235) (width 0.2) (layer "F.Cu") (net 8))
 (segment (start 122.5804 96.5454) (end 122.6058 96.52) (width 0.2) (layer "F.Cu") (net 8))
 (segment (start 122.6566 98.679) (end 122.555 98.7806) (width 0.2) (layer "F.Cu") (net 8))
 (segment (start 120.6119 99.1235) (end 120.9548 98.7806) (width 0.2) (layer "F.Cu") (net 8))
 (via (at 122.5804 96.5454) (size 0.6) (drill 0.3) (layers "F.Cu" "B.Cu") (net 8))
 (via (at 122.6566 98.679) (size 0.6) (drill 0.3) (layers "F.Cu" "B.Cu") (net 8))
 (segment (start 122.5804 96.5454) (end 122.5804 98.6028) (width 0.2) (layer "B.Cu") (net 8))
 (segment (start 122.5804 98.6028) (end 122.6566 98.679) (width 0.2) (layer "B.Cu") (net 8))
 (segment (start 120.7349 102.3874) (end 119.7926 102.3874) (width 0.2) (layer "F.Cu") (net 10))
 (segment (start 120.7349 102.3874) (end 124.9891 98.1332) (width 0.2) (layer "F.Cu") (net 10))
 (segment (start 119.7926 102.3874) (end 119.691 102.2858) (width 0.2) (layer "F.Cu") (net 10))
 (segment (start 120.6538 95.5332) (end 119.7864 94.6658) (width 0.2) (layer "F.Cu") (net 7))
 (segment (start 124.9891 95.5332) (end 120.6538 95.5332) (width 0.2) (layer "F.Cu") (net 7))
 (segment (start 119.7864 94.6658) (end 119.691 94.6658) (width 0.2) (layer "F.Cu") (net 7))
 (segment (start 121.5898 92.964) (end 121.5898 91.3892) (width 0.2) (layer "F.Cu") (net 5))
 (segment (start 119.7864 89.5858) (end 119.691 89.5858) (width 0.2) (layer "F.Cu") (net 5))
 (segment (start 124.9891 93.5832) (end 122.209 93.5832) (width 0.2) (layer "F.Cu") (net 5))
 (segment (start 122.209 93.5832) (end 121.5898 92.964) (width 0.2) (layer "F.Cu") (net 5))
 (segment (start 121.5898 91.3892) (end 119.7864 89.5858) (width 0.2) (layer "F.Cu") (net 5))
 (segment (start 129.2539 99.5934) (end 128.6256 99.4918) (width 0.2) (layer "F.Cu") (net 11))
 (segment (start 130.7141 98.1332) (end 129.2539 99.5934) (width 0.2) (layer "F.Cu") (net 11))
 (segment (start 128.6256 99.4918) (end 128.6764 99.5934) (width 0.2) (layer "F.Cu") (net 11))
 (via (at 128.6256 99.4918) (size 0.6) (drill 0.3) (layers "F.Cu" "B.Cu") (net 11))
 (segment (start 128.6256 99.4918) (end 129.8702 100.7364) (width 0.2) (layer "B.Cu") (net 11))
 (segment (start 135.8392 99.7966) (end 136.398 99.7966) (width 0.2) (layer "B.Cu") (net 11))
 (segment (start 129.8702 100.7364) (end 130.8354 100.7364) (width 0.2) (layer "B.Cu") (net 11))
 (segment (start 131.7752 99.7966) (end 135.8392 99.7966) (width 0.2) (layer "B.Cu") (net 11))
 (segment (start 130.8354 100.7364) (end 131.7752 99.7966) (width 0.2) (layer "B.Cu") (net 11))
 (segment (start 136.4742 99.7966) (end 136.652 99.6188) (width 0.2) (layer "B.Cu") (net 11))
 (segment (start 136.398 99.7966) (end 136.7282 99.4664) (width 0.2) (layer "B.Cu") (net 11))
 (segment (start 135.8392 99.7966) (end 136.4742 99.7966) (width 0.2) (layer "B.Cu") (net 11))
 (segment (start 131.826 102.5652) (end 132.3594 103.0986) (width 0.2) (layer "F.Cu") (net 12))
 (segment (start 135.2042 103.0986) (end 135.9027 102.4001) (width 0.2) (layer "F.Cu") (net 12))
 (segment (start 131.420056 97.4832) (end 131.826 97.889144) (width 0.2) (layer "F.Cu") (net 12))
 (segment (start 131.826 97.889144) (end 131.826 102.5652) (width 0.2) (layer "F.Cu") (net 12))
 (segment (start 136.3345 102.4001) (end 136.7282 102.0064) (width 0.2) (layer "F.Cu") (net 12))
 (segment (start 135.9027 102.4001) (end 136.3345 102.4001) (width 0.2) (layer "F.Cu") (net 12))
 (segment (start 130.7141 97.4832) (end 131.420056 97.4832) (width 0.2) (layer "F.Cu") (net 12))
 (segment (start 132.3594 103.0986) (end 135.2042 103.0986) (width 0.2) (layer "F.Cu") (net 12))
 (segment (start 136.144 102.1588) (end 136.652 102.1588) (width 0.2) (layer "F.Cu") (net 12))
 (segment (start 133.9096 94.2332) (end 135.6233 92.5195) (width 0.2) (layer "F.Cu") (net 13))
 (segment (start 136.1313 92.5195) (end 136.652 91.9988) (width 0.2) (layer "F.Cu") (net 13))
 (segment (start 135.8646 92.5195) (end 136.0551 92.5195) (width 0.2) (layer "F.Cu") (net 13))
 (segment (start 135.8646 92.5195) (end 136.1313 92.5195) (width 0.2) (layer "F.Cu") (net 13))
 (segment (start 136.0551 92.5195) (end 136.7282 91.8464) (width 0.2) (layer "F.Cu") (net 13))
 (segment (start 135.6233 92.5195) (end 135.8646 92.5195) (width 0.2) (layer "F.Cu") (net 13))
 (segment (start 130.7141 94.2332) (end 133.9096 94.2332) (width 0.2) (layer "F.Cu") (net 13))
 (segment (start 133.4008 89.6366) (end 135.509 89.6366) (width 0.2) (layer "F.Cu") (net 14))
 (segment (start 132.207 90.8304) (end 133.4008 89.6366) (width 0.2) (layer "F.Cu") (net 14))
 (segment (start 130.7141 93.5832) (end 131.791 93.5832) (width 0.2) (layer "F.Cu") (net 14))
 (segment (start 136.4742 89.6366) (end 136.652 89.4588) (width 0.2) (layer "F.Cu") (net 14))
 (segment (start 135.509 89.6366) (end 136.4742 89.6366) (width 0.2) (layer "F.Cu") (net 14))
 (segment (start 131.791 93.5832) (end 132.207 93.1672) (width 0.2) (layer "F.Cu") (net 14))
 (segment (start 135.509 89.6366) (end 136.398 89.6366) (width 0.2) (layer "F.Cu") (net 14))
 (segment (start 132.207 93.1672) (end 132.207 90.8304) (width 0.2) (layer "F.Cu") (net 14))
 (segment (start 136.398 89.6366) (end 136.7282 89.3064) (width 0.2) (layer "F.Cu") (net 14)))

